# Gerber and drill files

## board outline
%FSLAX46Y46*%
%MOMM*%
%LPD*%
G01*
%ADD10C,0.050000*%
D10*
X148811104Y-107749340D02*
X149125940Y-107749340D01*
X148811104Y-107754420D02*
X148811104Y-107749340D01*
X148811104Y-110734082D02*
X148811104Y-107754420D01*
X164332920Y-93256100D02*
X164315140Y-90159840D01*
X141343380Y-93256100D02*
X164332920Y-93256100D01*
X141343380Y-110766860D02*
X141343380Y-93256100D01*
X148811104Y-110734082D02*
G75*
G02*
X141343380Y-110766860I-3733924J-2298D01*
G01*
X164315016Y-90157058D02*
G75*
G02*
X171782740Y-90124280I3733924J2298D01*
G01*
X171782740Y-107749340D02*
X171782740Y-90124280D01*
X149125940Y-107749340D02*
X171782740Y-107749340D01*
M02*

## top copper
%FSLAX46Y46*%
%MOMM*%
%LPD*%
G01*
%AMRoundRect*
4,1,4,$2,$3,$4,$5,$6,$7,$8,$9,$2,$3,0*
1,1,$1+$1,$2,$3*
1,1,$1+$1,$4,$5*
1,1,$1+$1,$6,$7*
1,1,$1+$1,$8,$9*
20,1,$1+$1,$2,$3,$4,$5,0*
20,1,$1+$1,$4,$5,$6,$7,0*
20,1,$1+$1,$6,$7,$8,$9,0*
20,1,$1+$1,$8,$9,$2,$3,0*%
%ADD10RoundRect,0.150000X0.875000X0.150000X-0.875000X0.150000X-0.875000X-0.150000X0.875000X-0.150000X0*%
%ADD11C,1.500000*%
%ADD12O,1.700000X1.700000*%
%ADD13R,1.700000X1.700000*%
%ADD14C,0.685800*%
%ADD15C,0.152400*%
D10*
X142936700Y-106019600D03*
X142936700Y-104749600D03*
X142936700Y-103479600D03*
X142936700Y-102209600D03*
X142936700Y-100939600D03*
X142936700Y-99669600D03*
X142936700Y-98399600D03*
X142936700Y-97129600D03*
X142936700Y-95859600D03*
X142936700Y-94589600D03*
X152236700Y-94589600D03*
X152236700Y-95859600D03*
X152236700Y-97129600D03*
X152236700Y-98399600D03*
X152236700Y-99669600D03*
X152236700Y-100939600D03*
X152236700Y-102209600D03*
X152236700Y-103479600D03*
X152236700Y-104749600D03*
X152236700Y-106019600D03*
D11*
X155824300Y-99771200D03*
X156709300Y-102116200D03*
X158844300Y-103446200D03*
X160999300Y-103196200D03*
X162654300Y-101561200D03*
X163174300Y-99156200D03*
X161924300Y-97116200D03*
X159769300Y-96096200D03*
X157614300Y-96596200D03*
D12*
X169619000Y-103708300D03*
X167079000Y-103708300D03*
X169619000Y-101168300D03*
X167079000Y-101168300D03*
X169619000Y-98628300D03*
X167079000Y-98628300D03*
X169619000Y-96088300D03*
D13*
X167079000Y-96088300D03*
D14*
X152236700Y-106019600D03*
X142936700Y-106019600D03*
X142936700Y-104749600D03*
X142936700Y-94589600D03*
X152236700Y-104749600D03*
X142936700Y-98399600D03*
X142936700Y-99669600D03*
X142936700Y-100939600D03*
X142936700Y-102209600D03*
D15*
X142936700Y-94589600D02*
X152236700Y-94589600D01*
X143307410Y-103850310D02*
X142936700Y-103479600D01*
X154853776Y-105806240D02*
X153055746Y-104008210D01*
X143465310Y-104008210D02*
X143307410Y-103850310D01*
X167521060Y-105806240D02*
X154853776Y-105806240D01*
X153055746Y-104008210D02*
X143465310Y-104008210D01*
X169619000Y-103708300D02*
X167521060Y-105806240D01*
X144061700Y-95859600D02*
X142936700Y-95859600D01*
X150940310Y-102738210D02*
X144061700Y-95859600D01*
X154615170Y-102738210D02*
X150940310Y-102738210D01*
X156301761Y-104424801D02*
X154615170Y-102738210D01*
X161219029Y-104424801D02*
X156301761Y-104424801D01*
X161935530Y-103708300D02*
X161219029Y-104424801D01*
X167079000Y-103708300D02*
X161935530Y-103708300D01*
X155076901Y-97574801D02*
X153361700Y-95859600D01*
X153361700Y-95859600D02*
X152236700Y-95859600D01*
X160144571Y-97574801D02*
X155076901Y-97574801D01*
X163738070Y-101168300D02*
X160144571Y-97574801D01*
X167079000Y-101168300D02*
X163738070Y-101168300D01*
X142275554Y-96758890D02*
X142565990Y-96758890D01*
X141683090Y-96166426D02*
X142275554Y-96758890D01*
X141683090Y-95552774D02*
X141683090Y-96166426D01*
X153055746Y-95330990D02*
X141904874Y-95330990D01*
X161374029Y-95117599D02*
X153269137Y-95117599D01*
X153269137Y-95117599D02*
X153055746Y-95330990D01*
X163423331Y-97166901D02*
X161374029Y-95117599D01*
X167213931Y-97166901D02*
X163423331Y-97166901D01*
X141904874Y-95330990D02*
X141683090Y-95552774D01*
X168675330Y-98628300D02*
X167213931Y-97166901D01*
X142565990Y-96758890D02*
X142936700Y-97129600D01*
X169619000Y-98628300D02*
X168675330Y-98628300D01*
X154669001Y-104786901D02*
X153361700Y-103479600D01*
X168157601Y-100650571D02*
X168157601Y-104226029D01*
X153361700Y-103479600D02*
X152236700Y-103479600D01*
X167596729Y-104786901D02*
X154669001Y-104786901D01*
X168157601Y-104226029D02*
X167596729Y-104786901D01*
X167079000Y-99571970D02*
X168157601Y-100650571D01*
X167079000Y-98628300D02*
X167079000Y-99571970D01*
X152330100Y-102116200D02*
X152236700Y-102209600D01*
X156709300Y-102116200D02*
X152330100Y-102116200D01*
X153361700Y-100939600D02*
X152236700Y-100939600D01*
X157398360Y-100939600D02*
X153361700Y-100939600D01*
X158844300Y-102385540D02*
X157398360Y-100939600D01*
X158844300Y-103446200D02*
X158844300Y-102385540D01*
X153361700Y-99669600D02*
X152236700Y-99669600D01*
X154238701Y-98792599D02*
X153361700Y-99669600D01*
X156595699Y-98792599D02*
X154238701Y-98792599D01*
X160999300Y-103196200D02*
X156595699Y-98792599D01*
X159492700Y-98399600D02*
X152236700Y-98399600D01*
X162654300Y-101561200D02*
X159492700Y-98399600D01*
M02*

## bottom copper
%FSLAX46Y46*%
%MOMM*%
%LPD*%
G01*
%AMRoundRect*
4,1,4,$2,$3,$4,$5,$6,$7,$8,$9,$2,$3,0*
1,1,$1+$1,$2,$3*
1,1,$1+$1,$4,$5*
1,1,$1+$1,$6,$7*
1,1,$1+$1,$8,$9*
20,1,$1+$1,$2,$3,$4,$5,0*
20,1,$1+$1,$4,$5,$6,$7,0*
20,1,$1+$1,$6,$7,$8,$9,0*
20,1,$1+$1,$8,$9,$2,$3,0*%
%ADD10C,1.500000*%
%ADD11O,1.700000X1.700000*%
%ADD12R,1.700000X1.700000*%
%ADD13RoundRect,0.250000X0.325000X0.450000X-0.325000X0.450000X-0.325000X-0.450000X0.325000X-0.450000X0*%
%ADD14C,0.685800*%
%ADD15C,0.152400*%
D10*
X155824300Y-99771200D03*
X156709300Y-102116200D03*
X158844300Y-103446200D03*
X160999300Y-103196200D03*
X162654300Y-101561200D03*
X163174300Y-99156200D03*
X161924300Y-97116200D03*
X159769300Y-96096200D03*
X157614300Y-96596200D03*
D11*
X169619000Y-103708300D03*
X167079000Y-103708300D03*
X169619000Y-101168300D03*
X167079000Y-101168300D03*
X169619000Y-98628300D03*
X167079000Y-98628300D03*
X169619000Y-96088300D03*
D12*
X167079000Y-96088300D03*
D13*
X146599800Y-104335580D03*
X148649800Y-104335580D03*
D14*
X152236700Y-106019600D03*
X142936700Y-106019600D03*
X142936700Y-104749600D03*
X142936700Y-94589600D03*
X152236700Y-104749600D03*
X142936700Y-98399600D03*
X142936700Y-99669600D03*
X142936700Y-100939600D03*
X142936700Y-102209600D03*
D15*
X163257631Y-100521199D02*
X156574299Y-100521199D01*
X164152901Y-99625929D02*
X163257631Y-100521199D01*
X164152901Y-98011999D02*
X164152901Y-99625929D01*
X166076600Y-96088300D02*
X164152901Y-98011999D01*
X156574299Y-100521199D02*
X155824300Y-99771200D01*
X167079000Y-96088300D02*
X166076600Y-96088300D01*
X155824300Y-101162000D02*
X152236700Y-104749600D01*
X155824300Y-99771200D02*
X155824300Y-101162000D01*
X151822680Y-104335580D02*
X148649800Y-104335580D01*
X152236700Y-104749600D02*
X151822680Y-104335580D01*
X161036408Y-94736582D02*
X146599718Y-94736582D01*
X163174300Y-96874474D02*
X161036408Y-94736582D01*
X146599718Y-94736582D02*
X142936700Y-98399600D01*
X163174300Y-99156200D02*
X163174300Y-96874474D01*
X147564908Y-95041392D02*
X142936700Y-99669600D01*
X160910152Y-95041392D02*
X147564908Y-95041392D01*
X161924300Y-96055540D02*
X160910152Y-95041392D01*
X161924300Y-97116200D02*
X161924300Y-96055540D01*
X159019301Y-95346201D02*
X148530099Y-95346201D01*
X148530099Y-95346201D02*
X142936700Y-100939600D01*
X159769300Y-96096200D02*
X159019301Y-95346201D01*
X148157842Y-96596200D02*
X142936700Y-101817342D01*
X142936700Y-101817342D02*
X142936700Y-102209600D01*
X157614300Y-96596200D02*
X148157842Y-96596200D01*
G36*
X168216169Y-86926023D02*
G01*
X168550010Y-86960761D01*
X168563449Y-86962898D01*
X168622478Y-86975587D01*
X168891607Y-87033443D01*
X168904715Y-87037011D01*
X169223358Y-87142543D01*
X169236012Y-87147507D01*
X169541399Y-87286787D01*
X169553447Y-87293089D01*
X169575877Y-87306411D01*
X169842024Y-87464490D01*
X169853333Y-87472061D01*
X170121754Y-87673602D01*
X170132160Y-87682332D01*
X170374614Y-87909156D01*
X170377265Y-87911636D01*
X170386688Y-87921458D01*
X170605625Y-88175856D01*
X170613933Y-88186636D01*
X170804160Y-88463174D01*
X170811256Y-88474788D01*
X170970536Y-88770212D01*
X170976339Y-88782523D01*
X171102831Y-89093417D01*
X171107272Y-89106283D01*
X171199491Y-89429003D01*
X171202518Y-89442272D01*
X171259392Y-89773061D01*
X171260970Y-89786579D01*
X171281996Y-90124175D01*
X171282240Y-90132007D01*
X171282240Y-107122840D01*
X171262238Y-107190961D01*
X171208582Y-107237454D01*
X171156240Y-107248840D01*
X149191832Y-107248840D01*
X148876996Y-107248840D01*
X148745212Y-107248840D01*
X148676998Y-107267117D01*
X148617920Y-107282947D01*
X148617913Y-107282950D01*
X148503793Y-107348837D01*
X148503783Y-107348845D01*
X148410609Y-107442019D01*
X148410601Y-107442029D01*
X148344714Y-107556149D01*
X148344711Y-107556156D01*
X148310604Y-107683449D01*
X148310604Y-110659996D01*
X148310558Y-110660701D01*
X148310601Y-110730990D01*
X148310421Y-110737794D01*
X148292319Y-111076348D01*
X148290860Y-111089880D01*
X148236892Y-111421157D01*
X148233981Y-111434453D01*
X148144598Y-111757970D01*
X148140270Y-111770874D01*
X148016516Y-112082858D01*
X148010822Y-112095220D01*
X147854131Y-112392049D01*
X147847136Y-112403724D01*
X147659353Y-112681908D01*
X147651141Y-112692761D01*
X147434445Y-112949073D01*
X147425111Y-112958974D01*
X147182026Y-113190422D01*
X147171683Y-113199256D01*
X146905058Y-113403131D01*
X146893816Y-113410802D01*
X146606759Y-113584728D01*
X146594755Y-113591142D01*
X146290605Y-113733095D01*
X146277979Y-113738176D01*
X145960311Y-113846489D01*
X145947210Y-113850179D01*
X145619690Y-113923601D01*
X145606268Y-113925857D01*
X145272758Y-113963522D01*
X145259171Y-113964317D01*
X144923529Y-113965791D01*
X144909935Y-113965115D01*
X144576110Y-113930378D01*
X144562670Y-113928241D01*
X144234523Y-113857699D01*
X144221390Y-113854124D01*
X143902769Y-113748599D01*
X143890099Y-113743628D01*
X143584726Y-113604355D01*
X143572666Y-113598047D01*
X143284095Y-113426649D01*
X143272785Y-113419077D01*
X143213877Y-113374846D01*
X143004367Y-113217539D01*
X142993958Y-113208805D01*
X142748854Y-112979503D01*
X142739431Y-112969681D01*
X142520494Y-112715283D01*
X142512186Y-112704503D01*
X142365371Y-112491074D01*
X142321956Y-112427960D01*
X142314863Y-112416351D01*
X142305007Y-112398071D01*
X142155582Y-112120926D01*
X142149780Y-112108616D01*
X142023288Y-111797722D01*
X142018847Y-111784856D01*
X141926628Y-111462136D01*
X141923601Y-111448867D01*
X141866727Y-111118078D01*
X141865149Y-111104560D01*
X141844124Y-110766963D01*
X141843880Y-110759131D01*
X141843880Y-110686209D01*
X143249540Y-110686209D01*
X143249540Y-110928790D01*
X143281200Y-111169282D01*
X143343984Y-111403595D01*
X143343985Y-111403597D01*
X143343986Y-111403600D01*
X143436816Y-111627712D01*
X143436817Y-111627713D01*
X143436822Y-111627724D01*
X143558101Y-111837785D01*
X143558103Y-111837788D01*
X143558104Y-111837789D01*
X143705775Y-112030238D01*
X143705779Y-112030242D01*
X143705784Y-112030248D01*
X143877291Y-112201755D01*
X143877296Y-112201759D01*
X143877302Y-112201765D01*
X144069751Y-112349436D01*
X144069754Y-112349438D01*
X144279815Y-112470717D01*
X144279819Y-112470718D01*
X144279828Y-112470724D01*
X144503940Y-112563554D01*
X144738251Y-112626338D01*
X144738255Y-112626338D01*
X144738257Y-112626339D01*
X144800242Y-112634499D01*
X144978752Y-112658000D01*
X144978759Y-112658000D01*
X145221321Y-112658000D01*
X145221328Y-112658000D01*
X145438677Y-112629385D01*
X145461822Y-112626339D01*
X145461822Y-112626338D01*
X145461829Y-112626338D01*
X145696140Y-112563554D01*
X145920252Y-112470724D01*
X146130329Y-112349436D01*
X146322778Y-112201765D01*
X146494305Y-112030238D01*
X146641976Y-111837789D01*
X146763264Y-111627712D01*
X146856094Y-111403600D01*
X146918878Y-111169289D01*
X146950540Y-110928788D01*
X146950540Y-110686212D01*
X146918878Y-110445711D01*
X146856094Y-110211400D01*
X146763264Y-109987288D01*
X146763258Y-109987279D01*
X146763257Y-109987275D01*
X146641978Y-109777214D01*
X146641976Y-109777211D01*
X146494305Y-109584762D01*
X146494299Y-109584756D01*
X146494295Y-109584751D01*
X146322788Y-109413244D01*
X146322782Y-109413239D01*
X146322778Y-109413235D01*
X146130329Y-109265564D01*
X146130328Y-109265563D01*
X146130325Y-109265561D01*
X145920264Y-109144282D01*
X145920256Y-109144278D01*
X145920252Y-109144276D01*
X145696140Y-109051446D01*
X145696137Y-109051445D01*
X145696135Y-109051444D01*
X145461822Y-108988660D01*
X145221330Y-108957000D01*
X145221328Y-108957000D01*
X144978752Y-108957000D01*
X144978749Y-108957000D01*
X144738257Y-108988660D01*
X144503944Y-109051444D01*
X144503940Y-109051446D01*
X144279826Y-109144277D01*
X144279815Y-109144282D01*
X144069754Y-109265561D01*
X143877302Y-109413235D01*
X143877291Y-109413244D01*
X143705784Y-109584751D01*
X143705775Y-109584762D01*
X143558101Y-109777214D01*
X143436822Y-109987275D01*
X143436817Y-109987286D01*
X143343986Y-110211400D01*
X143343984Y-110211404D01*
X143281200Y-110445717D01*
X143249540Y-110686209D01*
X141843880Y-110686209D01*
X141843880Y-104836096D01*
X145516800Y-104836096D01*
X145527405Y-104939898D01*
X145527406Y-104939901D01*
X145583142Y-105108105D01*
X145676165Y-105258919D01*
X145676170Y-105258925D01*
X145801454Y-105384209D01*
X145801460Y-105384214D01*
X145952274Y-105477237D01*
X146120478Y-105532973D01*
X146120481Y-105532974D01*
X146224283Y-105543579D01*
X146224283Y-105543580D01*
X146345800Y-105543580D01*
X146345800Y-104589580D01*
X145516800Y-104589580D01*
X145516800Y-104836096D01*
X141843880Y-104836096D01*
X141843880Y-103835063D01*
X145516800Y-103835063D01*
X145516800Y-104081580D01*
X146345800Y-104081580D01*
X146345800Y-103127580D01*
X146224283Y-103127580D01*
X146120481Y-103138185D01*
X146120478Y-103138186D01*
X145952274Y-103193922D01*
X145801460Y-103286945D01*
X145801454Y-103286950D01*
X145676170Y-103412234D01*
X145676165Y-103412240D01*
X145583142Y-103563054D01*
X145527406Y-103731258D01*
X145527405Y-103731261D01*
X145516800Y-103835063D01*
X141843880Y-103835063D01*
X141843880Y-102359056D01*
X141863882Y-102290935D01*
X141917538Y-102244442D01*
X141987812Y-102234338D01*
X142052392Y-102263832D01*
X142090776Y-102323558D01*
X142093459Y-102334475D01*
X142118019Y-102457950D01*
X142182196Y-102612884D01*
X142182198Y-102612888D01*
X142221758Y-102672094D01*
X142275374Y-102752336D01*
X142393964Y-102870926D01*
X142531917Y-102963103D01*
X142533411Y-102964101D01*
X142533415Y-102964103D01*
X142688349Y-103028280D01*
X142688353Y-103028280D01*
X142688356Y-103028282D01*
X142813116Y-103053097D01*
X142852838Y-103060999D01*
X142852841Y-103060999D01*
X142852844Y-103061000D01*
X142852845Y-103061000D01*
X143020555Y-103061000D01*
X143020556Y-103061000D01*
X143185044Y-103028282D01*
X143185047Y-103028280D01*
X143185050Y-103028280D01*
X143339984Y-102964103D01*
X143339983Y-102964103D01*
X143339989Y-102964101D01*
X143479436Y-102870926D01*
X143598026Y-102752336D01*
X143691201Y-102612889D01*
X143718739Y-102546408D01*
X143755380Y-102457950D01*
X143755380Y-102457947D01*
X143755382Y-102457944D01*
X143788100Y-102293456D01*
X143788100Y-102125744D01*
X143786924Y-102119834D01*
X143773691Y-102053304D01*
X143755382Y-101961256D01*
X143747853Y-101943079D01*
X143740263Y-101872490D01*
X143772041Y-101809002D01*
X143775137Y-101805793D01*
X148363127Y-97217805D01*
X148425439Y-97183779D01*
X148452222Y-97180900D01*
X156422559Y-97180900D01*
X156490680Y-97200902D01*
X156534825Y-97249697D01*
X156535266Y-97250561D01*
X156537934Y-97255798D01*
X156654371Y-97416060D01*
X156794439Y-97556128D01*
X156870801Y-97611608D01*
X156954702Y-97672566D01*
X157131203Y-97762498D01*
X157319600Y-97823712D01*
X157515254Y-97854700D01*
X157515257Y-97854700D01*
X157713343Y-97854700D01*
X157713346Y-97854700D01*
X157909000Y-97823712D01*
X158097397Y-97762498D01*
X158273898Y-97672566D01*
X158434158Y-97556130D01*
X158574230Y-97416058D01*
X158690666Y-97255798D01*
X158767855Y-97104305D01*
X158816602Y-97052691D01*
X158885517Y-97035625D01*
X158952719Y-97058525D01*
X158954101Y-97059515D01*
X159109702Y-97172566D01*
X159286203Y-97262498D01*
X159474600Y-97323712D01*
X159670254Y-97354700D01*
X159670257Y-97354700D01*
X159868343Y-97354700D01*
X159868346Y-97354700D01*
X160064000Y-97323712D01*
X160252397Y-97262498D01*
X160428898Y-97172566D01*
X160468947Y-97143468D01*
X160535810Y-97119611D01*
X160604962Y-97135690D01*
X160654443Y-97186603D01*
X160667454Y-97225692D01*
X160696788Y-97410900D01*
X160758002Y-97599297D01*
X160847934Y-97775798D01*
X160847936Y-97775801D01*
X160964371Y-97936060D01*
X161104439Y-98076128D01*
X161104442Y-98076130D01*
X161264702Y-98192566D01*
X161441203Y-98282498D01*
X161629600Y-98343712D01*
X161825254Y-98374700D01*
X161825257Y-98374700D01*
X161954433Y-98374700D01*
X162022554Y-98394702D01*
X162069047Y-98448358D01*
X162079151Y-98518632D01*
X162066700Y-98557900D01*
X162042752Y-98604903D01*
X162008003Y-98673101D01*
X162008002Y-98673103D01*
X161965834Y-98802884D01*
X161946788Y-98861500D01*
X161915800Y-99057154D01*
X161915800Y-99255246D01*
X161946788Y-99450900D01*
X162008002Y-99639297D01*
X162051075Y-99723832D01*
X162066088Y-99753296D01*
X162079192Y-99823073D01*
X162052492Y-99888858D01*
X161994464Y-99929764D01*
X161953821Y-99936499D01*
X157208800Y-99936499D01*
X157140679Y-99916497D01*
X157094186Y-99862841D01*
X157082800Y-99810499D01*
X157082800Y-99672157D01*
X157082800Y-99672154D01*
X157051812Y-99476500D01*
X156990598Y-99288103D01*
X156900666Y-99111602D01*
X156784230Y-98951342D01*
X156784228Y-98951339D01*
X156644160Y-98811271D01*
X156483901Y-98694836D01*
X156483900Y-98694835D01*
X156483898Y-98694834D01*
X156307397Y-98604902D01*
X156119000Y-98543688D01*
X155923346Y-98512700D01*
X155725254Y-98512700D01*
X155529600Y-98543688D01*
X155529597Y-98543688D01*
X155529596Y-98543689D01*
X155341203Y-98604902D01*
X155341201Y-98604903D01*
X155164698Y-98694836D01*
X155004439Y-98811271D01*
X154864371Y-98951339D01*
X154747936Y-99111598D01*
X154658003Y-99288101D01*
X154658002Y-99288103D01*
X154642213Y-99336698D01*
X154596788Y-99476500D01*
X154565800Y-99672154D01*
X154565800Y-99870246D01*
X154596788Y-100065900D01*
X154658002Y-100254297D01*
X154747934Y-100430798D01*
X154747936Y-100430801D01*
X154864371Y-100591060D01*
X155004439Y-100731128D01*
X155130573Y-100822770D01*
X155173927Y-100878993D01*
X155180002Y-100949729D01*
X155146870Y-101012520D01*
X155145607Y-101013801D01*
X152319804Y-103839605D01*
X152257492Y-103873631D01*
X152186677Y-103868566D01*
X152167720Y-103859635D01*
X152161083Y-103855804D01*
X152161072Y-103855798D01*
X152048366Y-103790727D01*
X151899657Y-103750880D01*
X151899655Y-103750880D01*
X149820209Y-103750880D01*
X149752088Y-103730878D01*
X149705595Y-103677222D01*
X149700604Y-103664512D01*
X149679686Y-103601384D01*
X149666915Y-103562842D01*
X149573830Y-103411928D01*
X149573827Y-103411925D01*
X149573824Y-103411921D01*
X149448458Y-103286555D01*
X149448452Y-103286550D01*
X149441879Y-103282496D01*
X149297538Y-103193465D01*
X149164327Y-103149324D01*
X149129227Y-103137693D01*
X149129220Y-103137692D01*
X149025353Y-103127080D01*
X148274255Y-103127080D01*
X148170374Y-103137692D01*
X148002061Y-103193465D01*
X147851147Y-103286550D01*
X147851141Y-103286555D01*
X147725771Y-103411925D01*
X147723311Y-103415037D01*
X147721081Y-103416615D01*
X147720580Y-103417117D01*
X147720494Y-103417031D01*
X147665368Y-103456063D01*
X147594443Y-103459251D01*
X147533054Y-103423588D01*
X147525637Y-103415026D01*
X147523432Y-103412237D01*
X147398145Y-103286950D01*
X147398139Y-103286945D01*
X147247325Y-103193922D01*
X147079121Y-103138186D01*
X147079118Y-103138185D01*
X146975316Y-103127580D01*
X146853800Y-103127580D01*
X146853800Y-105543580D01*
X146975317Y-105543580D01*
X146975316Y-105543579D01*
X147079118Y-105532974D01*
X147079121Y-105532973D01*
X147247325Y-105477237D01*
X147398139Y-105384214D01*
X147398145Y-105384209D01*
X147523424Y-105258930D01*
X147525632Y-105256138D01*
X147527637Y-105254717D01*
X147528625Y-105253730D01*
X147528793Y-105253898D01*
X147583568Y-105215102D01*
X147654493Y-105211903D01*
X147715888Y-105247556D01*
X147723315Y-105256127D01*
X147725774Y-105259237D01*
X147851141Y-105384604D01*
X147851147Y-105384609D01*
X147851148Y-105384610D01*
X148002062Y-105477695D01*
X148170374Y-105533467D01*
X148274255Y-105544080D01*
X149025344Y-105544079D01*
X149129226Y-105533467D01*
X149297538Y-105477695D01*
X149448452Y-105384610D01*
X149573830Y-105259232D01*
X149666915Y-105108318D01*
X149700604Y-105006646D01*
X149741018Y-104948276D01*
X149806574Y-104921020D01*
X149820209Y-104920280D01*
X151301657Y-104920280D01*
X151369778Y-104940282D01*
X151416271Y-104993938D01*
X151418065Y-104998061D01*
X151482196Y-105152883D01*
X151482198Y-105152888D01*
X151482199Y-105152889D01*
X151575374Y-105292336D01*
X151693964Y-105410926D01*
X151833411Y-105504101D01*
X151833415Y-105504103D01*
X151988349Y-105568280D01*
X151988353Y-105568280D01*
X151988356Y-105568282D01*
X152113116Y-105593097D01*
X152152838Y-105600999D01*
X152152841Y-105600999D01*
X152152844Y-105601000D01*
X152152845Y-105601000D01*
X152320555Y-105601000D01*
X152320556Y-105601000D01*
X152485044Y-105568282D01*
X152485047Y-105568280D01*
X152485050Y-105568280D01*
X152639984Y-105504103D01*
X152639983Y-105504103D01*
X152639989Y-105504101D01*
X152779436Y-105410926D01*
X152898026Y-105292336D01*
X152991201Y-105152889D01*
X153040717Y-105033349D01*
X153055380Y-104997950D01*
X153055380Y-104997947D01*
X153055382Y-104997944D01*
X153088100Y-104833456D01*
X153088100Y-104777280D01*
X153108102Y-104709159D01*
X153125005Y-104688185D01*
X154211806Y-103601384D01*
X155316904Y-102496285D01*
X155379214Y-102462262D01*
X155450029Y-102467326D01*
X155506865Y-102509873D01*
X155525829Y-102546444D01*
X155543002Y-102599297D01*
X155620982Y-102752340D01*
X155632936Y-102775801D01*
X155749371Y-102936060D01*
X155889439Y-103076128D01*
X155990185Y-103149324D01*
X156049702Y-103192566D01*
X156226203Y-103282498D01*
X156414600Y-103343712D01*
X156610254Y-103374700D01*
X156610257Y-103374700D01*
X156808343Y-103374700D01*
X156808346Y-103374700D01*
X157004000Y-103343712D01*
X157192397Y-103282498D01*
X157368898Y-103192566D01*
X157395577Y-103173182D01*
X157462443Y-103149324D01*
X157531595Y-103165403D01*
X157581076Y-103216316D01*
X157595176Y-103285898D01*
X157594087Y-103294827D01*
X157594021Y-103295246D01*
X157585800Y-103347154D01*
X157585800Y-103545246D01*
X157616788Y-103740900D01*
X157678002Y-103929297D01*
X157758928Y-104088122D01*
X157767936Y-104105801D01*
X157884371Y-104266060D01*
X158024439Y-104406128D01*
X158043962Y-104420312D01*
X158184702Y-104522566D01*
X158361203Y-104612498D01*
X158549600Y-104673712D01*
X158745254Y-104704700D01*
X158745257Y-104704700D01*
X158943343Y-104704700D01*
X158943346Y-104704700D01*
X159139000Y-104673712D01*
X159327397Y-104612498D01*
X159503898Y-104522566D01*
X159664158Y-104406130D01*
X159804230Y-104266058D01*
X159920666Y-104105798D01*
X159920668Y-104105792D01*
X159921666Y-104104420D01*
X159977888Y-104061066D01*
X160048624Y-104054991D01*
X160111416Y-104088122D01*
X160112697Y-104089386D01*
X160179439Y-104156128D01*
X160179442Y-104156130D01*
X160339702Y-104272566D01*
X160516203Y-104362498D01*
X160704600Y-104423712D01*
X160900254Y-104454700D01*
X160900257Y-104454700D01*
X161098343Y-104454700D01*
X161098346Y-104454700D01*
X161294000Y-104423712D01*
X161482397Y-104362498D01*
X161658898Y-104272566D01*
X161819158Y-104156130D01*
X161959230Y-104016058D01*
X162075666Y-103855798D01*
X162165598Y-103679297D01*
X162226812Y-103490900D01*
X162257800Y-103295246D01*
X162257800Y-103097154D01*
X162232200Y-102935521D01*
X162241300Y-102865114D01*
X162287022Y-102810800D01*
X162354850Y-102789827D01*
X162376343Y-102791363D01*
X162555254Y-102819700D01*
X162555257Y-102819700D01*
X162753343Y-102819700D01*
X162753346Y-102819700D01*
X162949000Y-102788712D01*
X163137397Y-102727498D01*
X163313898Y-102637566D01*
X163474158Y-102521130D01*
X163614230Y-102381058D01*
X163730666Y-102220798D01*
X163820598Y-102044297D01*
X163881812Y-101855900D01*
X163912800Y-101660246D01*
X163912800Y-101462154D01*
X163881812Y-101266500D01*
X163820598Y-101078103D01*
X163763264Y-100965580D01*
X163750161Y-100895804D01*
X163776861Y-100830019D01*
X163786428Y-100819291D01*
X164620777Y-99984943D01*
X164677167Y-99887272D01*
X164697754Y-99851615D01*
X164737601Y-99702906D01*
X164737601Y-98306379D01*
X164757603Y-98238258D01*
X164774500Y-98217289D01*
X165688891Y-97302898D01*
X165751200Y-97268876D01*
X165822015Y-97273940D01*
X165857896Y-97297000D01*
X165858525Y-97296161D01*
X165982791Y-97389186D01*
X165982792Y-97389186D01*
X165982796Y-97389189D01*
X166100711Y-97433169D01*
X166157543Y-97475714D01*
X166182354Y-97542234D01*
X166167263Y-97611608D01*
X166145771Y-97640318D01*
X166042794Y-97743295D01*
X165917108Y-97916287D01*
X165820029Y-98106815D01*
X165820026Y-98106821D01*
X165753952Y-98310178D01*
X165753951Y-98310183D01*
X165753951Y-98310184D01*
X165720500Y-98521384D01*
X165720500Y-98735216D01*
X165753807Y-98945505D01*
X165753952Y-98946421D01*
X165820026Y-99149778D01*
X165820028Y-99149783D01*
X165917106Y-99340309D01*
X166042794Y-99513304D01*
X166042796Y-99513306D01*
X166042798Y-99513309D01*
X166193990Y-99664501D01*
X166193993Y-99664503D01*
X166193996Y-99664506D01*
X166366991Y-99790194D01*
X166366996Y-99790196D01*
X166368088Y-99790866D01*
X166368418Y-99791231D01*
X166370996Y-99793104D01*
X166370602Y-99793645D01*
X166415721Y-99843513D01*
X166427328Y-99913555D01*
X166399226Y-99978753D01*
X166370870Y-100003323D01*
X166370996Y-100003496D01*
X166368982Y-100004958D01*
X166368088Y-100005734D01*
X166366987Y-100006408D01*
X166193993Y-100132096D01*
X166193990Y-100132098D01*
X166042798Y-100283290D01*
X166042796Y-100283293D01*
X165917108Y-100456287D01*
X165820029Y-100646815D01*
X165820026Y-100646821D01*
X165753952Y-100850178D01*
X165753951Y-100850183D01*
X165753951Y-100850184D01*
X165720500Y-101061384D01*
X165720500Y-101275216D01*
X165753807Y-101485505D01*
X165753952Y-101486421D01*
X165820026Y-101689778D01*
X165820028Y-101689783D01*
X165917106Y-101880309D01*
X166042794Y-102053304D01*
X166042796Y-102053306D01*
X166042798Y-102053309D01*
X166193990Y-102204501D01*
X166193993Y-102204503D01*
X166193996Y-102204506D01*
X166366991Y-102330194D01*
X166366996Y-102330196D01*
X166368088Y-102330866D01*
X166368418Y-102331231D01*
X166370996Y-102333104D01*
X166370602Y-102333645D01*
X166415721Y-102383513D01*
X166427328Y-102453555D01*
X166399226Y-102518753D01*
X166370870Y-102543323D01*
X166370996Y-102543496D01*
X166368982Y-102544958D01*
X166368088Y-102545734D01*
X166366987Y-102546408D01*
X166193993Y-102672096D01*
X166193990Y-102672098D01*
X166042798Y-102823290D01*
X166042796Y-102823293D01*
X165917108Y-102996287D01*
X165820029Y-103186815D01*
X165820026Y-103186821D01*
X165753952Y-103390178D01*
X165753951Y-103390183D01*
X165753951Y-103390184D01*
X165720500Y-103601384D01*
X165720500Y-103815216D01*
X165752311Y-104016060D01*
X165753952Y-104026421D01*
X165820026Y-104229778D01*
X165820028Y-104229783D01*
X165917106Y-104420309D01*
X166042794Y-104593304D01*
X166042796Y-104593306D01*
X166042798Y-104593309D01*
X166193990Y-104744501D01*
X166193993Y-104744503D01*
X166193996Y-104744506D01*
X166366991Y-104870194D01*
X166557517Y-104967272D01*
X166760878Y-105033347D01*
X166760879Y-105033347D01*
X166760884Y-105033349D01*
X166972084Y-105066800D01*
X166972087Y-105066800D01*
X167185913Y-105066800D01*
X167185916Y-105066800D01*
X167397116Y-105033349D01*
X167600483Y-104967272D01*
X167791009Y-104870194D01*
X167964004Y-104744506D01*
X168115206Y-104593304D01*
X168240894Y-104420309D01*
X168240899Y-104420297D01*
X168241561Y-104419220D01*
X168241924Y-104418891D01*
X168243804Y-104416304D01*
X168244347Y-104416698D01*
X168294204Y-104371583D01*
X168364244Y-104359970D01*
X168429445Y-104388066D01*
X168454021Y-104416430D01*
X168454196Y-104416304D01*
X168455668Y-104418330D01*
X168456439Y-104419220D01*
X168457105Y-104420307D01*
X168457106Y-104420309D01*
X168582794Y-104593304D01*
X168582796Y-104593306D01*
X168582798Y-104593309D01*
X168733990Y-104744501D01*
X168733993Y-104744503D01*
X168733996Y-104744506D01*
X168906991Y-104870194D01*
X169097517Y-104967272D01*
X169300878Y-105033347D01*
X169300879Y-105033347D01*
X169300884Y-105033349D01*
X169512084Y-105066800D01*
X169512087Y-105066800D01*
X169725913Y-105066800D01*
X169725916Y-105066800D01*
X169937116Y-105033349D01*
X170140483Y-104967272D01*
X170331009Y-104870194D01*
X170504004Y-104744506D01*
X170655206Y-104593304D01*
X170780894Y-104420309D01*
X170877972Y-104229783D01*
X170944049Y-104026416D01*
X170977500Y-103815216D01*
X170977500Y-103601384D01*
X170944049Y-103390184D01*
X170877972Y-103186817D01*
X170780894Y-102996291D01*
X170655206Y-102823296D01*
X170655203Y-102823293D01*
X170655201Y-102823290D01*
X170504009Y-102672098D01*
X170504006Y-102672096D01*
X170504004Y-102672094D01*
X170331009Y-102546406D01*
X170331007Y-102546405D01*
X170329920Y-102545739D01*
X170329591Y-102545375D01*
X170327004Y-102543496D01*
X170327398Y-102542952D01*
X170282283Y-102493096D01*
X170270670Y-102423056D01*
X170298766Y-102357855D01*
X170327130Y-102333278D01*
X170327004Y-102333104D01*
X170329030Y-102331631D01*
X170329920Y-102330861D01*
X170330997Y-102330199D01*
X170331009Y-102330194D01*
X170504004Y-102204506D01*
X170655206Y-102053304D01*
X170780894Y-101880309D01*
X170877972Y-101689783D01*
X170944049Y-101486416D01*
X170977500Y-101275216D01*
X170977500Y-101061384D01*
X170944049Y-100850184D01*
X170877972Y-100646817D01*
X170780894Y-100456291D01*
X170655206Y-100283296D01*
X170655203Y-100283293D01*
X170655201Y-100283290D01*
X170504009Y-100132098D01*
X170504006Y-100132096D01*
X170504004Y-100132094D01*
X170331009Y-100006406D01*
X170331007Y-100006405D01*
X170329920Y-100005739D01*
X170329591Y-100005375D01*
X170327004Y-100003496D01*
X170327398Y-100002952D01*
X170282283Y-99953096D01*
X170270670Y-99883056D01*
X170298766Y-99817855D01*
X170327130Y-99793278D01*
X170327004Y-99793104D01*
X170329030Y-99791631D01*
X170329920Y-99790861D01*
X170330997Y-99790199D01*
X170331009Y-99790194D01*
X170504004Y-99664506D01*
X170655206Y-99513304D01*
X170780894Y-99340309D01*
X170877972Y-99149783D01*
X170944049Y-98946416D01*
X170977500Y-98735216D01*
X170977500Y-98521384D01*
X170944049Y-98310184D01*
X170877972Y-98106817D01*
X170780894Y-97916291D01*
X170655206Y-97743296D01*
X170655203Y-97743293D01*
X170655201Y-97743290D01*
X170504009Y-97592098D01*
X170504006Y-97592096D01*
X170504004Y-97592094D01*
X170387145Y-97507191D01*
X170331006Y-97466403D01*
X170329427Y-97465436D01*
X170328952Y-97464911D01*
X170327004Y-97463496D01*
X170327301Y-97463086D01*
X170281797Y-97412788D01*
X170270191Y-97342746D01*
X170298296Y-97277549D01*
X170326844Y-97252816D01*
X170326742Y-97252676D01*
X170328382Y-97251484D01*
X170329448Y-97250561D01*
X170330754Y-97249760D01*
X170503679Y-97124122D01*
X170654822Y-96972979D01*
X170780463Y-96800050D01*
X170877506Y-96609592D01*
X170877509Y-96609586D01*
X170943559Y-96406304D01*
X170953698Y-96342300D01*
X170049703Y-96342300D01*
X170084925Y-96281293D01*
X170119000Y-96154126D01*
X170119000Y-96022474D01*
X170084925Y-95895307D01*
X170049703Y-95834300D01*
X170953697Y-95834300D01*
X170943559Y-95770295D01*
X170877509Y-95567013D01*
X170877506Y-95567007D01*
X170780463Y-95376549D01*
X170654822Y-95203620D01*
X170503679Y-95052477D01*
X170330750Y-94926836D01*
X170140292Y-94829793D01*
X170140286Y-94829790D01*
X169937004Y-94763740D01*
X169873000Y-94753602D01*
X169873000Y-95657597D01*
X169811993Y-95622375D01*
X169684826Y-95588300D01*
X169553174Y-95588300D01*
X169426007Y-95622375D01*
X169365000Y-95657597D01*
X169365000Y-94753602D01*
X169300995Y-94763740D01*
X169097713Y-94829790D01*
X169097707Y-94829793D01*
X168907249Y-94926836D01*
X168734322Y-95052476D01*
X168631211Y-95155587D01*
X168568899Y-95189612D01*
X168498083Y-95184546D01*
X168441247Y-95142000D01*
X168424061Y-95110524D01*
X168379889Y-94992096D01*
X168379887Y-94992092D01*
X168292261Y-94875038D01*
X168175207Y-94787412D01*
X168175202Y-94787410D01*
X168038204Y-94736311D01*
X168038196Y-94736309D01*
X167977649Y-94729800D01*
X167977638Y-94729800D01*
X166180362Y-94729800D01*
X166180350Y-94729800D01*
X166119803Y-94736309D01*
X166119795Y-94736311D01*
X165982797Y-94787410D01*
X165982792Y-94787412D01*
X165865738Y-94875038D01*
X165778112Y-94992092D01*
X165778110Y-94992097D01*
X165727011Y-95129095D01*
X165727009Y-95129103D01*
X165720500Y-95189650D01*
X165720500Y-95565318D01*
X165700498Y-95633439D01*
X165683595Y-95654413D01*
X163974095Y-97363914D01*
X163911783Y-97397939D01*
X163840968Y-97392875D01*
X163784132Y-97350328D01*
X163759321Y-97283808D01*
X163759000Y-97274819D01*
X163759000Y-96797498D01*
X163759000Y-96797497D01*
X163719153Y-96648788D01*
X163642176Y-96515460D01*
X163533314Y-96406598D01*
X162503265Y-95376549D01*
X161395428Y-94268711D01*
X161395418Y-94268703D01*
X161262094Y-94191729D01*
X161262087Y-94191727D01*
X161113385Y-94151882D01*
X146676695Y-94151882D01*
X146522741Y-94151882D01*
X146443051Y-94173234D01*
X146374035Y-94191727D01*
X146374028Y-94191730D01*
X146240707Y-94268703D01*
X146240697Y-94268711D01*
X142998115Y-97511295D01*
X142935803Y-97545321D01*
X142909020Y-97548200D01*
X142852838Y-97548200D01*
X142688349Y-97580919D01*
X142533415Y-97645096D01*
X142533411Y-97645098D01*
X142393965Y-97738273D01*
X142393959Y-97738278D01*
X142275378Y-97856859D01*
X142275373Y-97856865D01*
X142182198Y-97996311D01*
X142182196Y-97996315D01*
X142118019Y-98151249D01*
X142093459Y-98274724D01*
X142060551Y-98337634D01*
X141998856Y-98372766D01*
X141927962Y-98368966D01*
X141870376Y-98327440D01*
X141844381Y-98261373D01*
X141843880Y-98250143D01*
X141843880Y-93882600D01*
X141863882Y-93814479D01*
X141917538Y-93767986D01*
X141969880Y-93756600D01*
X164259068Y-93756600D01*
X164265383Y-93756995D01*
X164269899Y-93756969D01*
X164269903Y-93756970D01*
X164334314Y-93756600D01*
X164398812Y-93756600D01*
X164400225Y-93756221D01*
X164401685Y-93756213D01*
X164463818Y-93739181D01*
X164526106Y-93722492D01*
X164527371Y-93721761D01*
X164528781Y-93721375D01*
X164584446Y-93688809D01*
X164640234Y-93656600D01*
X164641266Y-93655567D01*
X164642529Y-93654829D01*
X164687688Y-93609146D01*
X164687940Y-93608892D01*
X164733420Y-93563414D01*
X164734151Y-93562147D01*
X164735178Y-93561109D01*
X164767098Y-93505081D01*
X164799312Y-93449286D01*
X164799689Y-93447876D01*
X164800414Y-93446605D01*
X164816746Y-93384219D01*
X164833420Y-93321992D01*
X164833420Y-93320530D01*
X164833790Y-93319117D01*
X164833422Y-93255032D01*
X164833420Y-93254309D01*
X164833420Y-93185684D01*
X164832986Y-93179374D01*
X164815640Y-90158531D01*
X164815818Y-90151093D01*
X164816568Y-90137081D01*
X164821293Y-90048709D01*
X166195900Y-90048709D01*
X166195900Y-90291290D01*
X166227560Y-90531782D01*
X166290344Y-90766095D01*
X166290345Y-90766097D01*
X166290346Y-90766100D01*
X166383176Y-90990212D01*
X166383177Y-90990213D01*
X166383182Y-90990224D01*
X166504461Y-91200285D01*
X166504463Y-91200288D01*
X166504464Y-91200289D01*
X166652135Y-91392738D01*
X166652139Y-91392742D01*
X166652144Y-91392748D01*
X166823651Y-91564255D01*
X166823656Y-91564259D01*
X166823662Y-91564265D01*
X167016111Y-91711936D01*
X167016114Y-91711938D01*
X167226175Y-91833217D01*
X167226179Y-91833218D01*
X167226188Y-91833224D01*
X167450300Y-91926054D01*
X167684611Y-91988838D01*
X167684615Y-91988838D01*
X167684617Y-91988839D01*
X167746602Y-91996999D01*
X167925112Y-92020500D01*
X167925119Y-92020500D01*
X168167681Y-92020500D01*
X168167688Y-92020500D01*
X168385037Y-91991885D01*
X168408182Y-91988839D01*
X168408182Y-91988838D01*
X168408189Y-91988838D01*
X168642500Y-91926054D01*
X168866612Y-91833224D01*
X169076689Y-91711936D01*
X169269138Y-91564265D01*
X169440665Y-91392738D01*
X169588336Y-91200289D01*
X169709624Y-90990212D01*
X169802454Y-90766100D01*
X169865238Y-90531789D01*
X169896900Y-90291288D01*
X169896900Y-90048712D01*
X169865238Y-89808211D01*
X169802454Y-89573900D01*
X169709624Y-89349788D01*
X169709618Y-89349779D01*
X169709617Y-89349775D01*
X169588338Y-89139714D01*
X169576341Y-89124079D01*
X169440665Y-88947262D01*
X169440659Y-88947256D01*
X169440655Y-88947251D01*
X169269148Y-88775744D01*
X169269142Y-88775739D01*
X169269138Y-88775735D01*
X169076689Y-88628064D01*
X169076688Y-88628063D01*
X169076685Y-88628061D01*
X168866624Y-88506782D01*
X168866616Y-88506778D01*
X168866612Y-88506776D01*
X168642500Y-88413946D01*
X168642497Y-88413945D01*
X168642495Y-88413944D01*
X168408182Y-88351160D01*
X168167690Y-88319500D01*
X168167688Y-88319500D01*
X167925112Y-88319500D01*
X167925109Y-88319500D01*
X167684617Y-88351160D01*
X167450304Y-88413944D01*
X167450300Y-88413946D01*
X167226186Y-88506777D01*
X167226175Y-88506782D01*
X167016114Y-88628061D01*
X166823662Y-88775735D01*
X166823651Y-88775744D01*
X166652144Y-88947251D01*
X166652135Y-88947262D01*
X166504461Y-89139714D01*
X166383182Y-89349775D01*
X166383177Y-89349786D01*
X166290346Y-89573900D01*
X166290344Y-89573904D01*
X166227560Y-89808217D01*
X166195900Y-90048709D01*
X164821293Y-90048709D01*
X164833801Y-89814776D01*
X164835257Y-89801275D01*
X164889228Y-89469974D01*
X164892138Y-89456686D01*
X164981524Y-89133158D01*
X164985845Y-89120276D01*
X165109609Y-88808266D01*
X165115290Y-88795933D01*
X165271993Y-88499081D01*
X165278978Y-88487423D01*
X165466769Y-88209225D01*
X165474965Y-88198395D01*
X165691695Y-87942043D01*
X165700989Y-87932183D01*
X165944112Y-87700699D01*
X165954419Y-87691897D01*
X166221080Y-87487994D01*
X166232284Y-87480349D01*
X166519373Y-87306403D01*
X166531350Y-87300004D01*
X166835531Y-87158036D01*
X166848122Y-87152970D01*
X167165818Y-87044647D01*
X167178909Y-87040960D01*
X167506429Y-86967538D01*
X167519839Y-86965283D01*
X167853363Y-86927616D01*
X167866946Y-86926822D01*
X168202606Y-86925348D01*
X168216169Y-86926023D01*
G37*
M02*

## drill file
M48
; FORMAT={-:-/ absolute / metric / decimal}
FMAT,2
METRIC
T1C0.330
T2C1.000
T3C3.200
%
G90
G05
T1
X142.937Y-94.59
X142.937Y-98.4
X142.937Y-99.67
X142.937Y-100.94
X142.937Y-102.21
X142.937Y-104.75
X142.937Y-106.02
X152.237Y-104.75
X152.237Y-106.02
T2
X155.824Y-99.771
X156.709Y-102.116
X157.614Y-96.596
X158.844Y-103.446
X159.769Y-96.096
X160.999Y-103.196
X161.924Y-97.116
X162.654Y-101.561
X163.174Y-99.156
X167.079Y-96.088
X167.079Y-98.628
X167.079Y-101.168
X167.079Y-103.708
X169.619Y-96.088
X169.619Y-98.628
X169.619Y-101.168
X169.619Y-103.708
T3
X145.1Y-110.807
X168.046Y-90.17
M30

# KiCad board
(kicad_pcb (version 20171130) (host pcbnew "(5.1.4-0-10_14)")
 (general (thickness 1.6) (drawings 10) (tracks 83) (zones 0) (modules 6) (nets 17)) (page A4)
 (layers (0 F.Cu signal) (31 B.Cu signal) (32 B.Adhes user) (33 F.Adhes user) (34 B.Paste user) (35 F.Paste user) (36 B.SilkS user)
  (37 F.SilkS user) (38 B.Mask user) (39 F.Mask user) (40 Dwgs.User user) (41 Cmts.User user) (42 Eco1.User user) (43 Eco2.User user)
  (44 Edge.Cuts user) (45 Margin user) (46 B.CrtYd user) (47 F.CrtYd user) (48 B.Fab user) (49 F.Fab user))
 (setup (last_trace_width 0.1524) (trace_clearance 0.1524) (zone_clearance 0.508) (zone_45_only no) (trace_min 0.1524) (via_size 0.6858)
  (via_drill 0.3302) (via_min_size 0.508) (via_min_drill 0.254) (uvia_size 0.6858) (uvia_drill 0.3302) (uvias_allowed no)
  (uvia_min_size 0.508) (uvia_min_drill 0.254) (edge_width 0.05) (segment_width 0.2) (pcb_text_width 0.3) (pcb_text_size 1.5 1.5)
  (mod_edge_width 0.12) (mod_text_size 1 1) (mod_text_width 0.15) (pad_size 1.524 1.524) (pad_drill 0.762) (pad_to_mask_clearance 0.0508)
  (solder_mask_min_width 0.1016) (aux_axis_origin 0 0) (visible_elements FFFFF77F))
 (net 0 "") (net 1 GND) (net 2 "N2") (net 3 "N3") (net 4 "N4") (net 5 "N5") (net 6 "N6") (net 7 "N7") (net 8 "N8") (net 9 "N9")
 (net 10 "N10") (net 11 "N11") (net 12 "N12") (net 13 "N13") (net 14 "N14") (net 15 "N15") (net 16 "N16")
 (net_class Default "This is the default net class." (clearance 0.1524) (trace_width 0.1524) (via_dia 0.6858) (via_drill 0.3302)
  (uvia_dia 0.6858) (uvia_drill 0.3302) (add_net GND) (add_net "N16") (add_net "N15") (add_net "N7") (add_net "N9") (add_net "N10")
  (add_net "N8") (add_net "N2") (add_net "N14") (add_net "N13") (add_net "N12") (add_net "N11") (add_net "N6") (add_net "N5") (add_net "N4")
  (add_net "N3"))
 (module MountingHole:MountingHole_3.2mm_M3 (layer F.Cu) (at 145.10004 110.8075)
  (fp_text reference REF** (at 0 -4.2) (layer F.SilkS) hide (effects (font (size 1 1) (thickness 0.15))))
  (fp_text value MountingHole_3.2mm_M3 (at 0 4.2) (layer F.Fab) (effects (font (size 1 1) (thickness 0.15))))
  (pad 1 np_thru_hole circle (at 0 0) (size 3.2 3.2) (drill 3.2) (layers *.Cu *.Mask)))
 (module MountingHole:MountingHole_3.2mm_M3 (layer F.Cu) (at 168.0464 90.17)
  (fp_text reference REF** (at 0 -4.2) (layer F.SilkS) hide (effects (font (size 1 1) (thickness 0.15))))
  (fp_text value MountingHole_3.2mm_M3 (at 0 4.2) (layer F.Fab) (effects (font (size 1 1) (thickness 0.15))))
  (pad 1 np_thru_hole circle (at 0 0) (size 3.2 3.2) (drill 3.2) (layers *.Cu *.Mask)))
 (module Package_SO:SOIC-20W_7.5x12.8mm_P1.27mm (layer F.Cu) (at 147.5867 100.3046 180)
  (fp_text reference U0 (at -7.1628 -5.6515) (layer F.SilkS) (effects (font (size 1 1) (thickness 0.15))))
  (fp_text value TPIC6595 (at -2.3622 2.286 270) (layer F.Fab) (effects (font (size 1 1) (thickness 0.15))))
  (pad 20 smd roundrect (at 4.65 -5.715 180) (size 2.05 0.6) (layers F.Cu F.Paste F.Mask) (roundrect_rratio 0.25) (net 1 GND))
  (pad 19 smd roundrect (at 4.65 -4.445 180) (size 2.05 0.6) (layers F.Cu F.Paste F.Mask) (roundrect_rratio 0.25) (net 1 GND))
  (pad 18 smd roundrect (at 4.65 -3.175 180) (size 2.05 0.6) (layers F.Cu F.Paste F.Mask) (roundrect_rratio 0.25) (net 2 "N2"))
  (pad 17 smd roundrect (at 4.65 -1.905 180) (size 2.05 0.6) (layers F.Cu F.Paste F.Mask) (roundrect_rratio 0.25) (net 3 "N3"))
  (pad 16 smd roundrect (at 4.65 -0.635 180) (size 2.05 0.6) (layers F.Cu F.Paste F.Mask) (roundrect_rratio 0.25) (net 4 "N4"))
  (pad 15 smd roundrect (at 4.65 0.635 180) (size 2.05 0.6) (layers F.Cu F.Paste F.Mask) (roundrect_rratio 0.25) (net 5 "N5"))
  (pad 14 smd roundrect (at 4.65 1.905 180) (size 2.05 0.6) (layers F.Cu F.Paste F.Mask) (roundrect_rratio 0.25) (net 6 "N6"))
  (pad 13 smd roundrect (at 4.65 3.175 180) (size 2.05 0.6) (layers F.Cu F.Paste F.Mask) (roundrect_rratio 0.25) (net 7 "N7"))
  (pad 12 smd roundrect (at 4.65 4.445 180) (size 2.05 0.6) (layers F.Cu F.Paste F.Mask) (roundrect_rratio 0.25) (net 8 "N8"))
  (pad 11 smd roundrect (at 4.65 5.715 180) (size 2.05 0.6) (layers F.Cu F.Paste F.Mask) (roundrect_rratio 0.25) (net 1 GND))
  (pad 10 smd roundrect (at -4.65 5.715 180) (size 2.05 0.6) (layers F.Cu F.Paste F.Mask) (roundrect_rratio 0.25) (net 1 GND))
  (pad 9 smd roundrect (at -4.65 4.445 180) (size 2.05 0.6) (layers F.Cu F.Paste F.Mask) (roundrect_rratio 0.25) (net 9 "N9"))
  (pad 8 smd roundrect (at -4.65 3.175 180) (size 2.05 0.6) (layers F.Cu F.Paste F.Mask) (roundrect_rratio 0.25) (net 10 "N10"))
  (pad 7 smd roundrect (at -4.65 1.905 180) (size 2.05 0.6) (layers F.Cu F.Paste F.Mask) (roundrect_rratio 0.25) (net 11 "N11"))
  (pad 6 smd roundrect (at -4.65 0.635 180) (size 2.05 0.6) (layers F.Cu F.Paste F.Mask) (roundrect_rratio 0.25) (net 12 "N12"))
  (pad 5 smd roundrect (at -4.65 -0.635 180) (size 2.05 0.6) (layers F.Cu F.Paste F.Mask) (roundrect_rratio 0.25) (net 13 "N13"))
  (pad 4 smd roundrect (at -4.65 -1.905 180) (size 2.05 0.6) (layers F.Cu F.Paste F.Mask) (roundrect_rratio 0.25) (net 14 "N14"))
  (pad 3 smd roundrect (at -4.65 -3.175 180) (size 2.05 0.6) (layers F.Cu F.Paste F.Mask) (roundrect_rratio 0.25) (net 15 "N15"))
  (pad 2 smd roundrect (at -4.65 -4.445 180) (size 2.05 0.6) (layers F.Cu F.Paste F.Mask) (roundrect_rratio 0.25) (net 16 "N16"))
  (pad 1 smd roundrect (at -4.65 -5.715 180) (size 2.05 0.6) (layers F.Cu F.Paste F.Mask) (roundrect_rratio 0.25) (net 1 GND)))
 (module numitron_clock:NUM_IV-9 (layer F.Cu) (at 159.4993 99.7712 270)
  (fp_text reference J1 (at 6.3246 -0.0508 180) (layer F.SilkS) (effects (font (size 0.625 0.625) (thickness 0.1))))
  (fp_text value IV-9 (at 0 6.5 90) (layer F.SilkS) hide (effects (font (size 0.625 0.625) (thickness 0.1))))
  (pad 1 thru_hole circle (at 0 3.675 270) (size 1.5 1.5) (drill 1) (layers *.Cu *.Mask F.SilkS) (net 16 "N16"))
  (pad 2 thru_hole circle (at 2.345 2.79 270) (size 1.5 1.5) (drill 1) (layers *.Cu *.Mask F.SilkS) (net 14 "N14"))
  (pad 3 thru_hole circle (at 3.675 0.655 270) (size 1.5 1.5) (drill 1) (layers *.Cu *.Mask F.SilkS) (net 13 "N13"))
  (pad 4 thru_hole circle (at 3.425 -1.5 270) (size 1.5 1.5) (drill 1) (layers *.Cu *.Mask F.SilkS) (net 12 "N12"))
  (pad 5 thru_hole circle (at 1.79 -3.155 270) (size 1.5 1.5) (drill 1) (layers *.Cu *.Mask F.SilkS) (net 11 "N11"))
  (pad 6 thru_hole circle (at -0.615 -3.675 270) (size 1.5 1.5) (drill 1) (layers *.Cu *.Mask F.SilkS) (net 6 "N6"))
  (pad 7 thru_hole circle (at -2.655 -2.425 270) (size 1.5 1.5) (drill 1) (layers *.Cu *.Mask F.SilkS) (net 5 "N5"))
  (pad 8 thru_hole circle (at -3.675 -0.27 270) (size 1.5 1.5) (drill 1) (layers *.Cu *.Mask F.SilkS) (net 4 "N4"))
  (pad 9 thru_hole circle (at -3.175 1.885 270) (size 1.5 1.5) (drill 1) (layers *.Cu *.Mask F.SilkS) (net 3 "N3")))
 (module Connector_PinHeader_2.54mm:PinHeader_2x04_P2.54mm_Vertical (layer F.Cu) (at 167.079 96.0883)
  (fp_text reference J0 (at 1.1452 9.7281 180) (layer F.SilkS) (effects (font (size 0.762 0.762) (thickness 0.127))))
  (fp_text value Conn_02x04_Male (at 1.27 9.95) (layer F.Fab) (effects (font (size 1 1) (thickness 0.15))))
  (pad 8 thru_hole oval (at 2.54 7.62) (size 1.7 1.7) (drill 1) (layers *.Cu *.Mask) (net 2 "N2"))
  (pad 7 thru_hole oval (at 0 7.62) (size 1.7 1.7) (drill 1) (layers *.Cu *.Mask) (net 8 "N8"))
  (pad 6 thru_hole oval (at 2.54 5.08) (size 1.7 1.7) (drill 1) (layers *.Cu *.Mask) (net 10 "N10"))
  (pad 5 thru_hole oval (at 0 5.08) (size 1.7 1.7) (drill 1) (layers *.Cu *.Mask) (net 9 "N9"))
  (pad 4 thru_hole oval (at 2.54 2.54) (size 1.7 1.7) (drill 1) (layers *.Cu *.Mask) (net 7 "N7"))
  (pad 3 thru_hole oval (at 0 2.54) (size 1.7 1.7) (drill 1) (layers *.Cu *.Mask) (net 15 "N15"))
  (pad 2 thru_hole oval (at 2.54 0) (size 1.7 1.7) (drill 1) (layers *.Cu *.Mask) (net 1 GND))
  (pad 1 thru_hole rect (at 0 0) (size 1.7 1.7) (drill 1) (layers *.Cu *.Mask) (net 16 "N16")))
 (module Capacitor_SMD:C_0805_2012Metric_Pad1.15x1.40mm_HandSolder (layer B.Cu) (at 147.6248 104.33558 180)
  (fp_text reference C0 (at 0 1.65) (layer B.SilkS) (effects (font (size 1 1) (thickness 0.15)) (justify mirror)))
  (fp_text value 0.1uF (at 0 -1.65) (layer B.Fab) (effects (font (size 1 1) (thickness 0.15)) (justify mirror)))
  (pad 2 smd roundrect (at 1.025 0 180) (size 1.15 1.4) (layers B.Cu B.Paste B.Mask) (roundrect_rratio 0.217391) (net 1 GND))
  (pad 1 smd roundrect (at -1.025 0 180) (size 1.15 1.4) (layers B.Cu B.Paste B.Mask) (roundrect_rratio 0.217391) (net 16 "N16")))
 (gr_line (start 148.811104 107.74934) (end 149.12594 107.74934) (layer Edge.Cuts) (width 0.05))
 (gr_line (start 148.811104 107.75442) (end 148.811104 107.74934) (layer Edge.Cuts) (width 0.05))
 (gr_line (start 148.811104 110.734082) (end 148.811104 107.75442) (layer Edge.Cuts) (width 0.05))
 (gr_line (start 164.33292 93.2561) (end 164.31514 90.15984) (layer Edge.Cuts) (width 0.05))
 (gr_line (start 141.34338 93.2561) (end 164.33292 93.2561) (layer Edge.Cuts) (width 0.05))
 (gr_line (start 141.34338 110.76686) (end 141.34338 93.2561) (layer Edge.Cuts) (width 0.05))
 (gr_arc (start 145.07718 110.73638) (end 141.34338 110.76686) (angle -179.567545) (layer Edge.Cuts) (width 0.05))
 (gr_arc (start 168.04894 90.15476) (end 171.78274 90.12428) (angle -179.567545) (layer Edge.Cuts) (width 0.05))
 (gr_line (start 171.78274 107.74934) (end 171.78274 90.12428) (layer Edge.Cuts) (width 0.05))
 (gr_line (start 149.12594 107.74934) (end 171.78274 107.74934) (layer Edge.Cuts) (width 0.05))
 (via (at 152.2367 106.0196) (size 0.6858) (drill 0.3302) (layers F.Cu B.Cu) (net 1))
 (via (at 142.9367 106.0196) (size 0.6858) (drill 0.3302) (layers F.Cu B.Cu) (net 1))
 (via (at 142.9367 104.7496) (size 0.6858) (drill 0.3302) (layers F.Cu B.Cu) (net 1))
 (via (at 142.9367 94.5896) (size 0.6858) (drill 0.3302) (layers F.Cu B.Cu) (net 1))
 (segment (start 142.9367 94.5896) (end 152.2367 94.5896) (width 0.1524) (layer F.Cu) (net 1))
 (via (at 152.2367 104.7496) (size 0.6858) (drill 0.3302) (layers F.Cu B.Cu) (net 16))
 (segment (start 163.257631 100.521199) (end 156.574299 100.521199) (width 0.1524) (layer B.Cu) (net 16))
 (segment (start 164.152901 99.625929) (end 163.257631 100.521199) (width 0.1524) (layer B.Cu) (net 16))
 (segment (start 164.152901 98.011999) (end 164.152901 99.625929) (width 0.1524) (layer B.Cu) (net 16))
 (segment (start 166.0766 96.0883) (end 164.152901 98.011999) (width 0.1524) (layer B.Cu) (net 16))
 (segment (start 156.574299 100.521199) (end 155.8243 99.7712) (width 0.1524) (layer B.Cu) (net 16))
 (segment (start 167.079 96.0883) (end 166.0766 96.0883) (width 0.1524) (layer B.Cu) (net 16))
 (segment (start 155.8243 101.162) (end 152.2367 104.7496) (width 0.1524) (layer B.Cu) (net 16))
 (segment (start 155.8243 99.7712) (end 155.8243 101.162) (width 0.1524) (layer B.Cu) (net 16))
 (segment (start 151.82268 104.33558) (end 148.6498 104.33558) (width 0.1524) (layer B.Cu) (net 16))
 (segment (start 152.2367 104.7496) (end 151.82268 104.33558) (width 0.1524) (layer B.Cu) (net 16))
 (segment (start 143.30741 103.85031) (end 142.9367 103.4796) (width 0.1524) (layer F.Cu) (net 2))
 (segment (start 154.853776 105.80624) (end 153.055746 104.00821) (width 0.1524) (layer F.Cu) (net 2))
 (segment (start 143.46531 104.00821) (end 143.30741 103.85031) (width 0.1524) (layer F.Cu) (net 2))
 (segment (start 167.52106 105.80624) (end 154.853776 105.80624) (width 0.1524) (layer F.Cu) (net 2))
 (segment (start 153.055746 104.00821) (end 143.46531 104.00821) (width 0.1524) (layer F.Cu) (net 2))
 (segment (start 169.619 103.7083) (end 167.52106 105.80624) (width 0.1524) (layer F.Cu) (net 2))
 (segment (start 144.0617 95.8596) (end 142.9367 95.8596) (width 0.1524) (layer F.Cu) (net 8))
 (segment (start 150.94031 102.73821) (end 144.0617 95.8596) (width 0.1524) (layer F.Cu) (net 8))
 (segment (start 154.61517 102.73821) (end 150.94031 102.73821) (width 0.1524) (layer F.Cu) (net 8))
 (segment (start 156.301761 104.424801) (end 154.61517 102.73821) (width 0.1524) (layer F.Cu) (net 8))
 (segment (start 161.219029 104.424801) (end 156.301761 104.424801) (width 0.1524) (layer F.Cu) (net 8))
 (segment (start 161.93553 103.7083) (end 161.219029 104.424801) (width 0.1524) (layer F.Cu) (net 8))
 (segment (start 167.079 103.7083) (end 161.93553 103.7083) (width 0.1524) (layer F.Cu) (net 8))
 (segment (start 155.076901 97.574801) (end 153.3617 95.8596) (width 0.1524) (layer F.Cu) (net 9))
 (segment (start 153.3617 95.8596) (end 152.2367 95.8596) (width 0.1524) (layer F.Cu) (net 9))
 (segment (start 160.144571 97.574801) (end 155.076901 97.574801) (width 0.1524) (layer F.Cu) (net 9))
 (segment (start 163.73807 101.1683) (end 160.144571 97.574801) (width 0.1524) (layer F.Cu) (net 9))
 (segment (start 167.079 101.1683) (end 163.73807 101.1683) (width 0.1524) (layer F.Cu) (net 9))
 (segment (start 142.275554 96.75889) (end 142.56599 96.75889) (width 0.1524) (layer F.Cu) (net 7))
 (segment (start 141.68309 96.166426) (end 142.275554 96.75889) (width 0.1524) (layer F.Cu) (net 7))
 (segment (start 141.68309 95.552774) (end 141.68309 96.166426) (width 0.1524) (layer F.Cu) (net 7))
 (segment (start 153.055746 95.33099) (end 141.904874 95.33099) (width 0.1524) (layer F.Cu) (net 7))
 (segment (start 161.374029 95.117599) (end 153.269137 95.117599) (width 0.1524) (layer F.Cu) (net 7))
 (segment (start 153.269137 95.117599) (end 153.055746 95.33099) (width 0.1524) (layer F.Cu) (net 7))
 (segment (start 163.423331 97.166901) (end 161.374029 95.117599) (width 0.1524) (layer F.Cu) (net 7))
 (segment (start 167.213931 97.166901) (end 163.423331 97.166901) (width 0.1524) (layer F.Cu) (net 7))
 (segment (start 141.904874 95.33099) (end 141.68309 95.552774) (width 0.1524) (layer F.Cu) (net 7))
 (segment (start 168.67533 98.6283) (end 167.213931 97.166901) (width 0.1524) (layer F.Cu) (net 7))
 (segment (start 142.56599 96.75889) (end 142.9367 97.1296) (width 0.1524) (layer F.Cu) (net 7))
 (segment (start 169.619 98.6283) (end 168.67533 98.6283) (width 0.1524) (layer F.Cu) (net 7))
 (segment (start 154.669001 104.786901) (end 153.3617 103.4796) (width 0.1524) (layer F.Cu) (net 15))
 (segment (start 168.157601 100.650571) (end 168.157601 104.226029) (width 0.1524) (layer F.Cu) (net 15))
 (segment (start 153.3617 103.4796) (end 152.2367 103.4796) (width 0.1524) (layer F.Cu) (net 15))
 (segment (start 167.596729 104.786901) (end 154.669001 104.786901) (width 0.1524) (layer F.Cu) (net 15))
 (segment (start 168.157601 104.226029) (end 167.596729 104.786901) (width 0.1524) (layer F.Cu) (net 15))
 (segment (start 167.079 99.57197) (end 168.157601 100.650571) (width 0.1524) (layer F.Cu) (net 15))
 (segment (start 167.079 98.6283) (end 167.079 99.57197) (width 0.1524) (layer F.Cu) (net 15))
 (segment (start 152.3301 102.1162) (end 152.2367 102.2096) (width 0.1524) (layer F.Cu) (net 14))
 (segment (start 156.7093 102.1162) (end 152.3301 102.1162) (width 0.1524) (layer F.Cu) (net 14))
 (segment (start 153.3617 100.9396) (end 152.2367 100.9396) (width 0.1524) (layer F.Cu) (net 13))
 (segment (start 157.39836 100.9396) (end 153.3617 100.9396) (width 0.1524) (layer F.Cu) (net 13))
 (segment (start 158.8443 102.38554) (end 157.39836 100.9396) (width 0.1524) (layer F.Cu) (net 13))
 (segment (start 158.8443 103.4462) (end 158.8443 102.38554) (width 0.1524) (layer F.Cu) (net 13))
 (segment (start 153.3617 99.6696) (end 152.2367 99.6696) (width 0.1524) (layer F.Cu) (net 12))
 (segment (start 154.238701 98.792599) (end 153.3617 99.6696) (width 0.1524) (layer F.Cu) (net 12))
 (segment (start 156.595699 98.792599) (end 154.238701 98.792599) (width 0.1524) (layer F.Cu) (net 12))
 (segment (start 160.9993 103.1962) (end 156.595699 98.792599) (width 0.1524) (layer F.Cu) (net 12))
 (segment (start 159.4927 98.3996) (end 152.2367 98.3996) (width 0.1524) (layer F.Cu) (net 11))
 (segment (start 162.6543 101.5612) (end 159.4927 98.3996) (width 0.1524) (layer F.Cu) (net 11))
 (segment (start 161.036408 94.736582) (end 146.599718 94.736582) (width 0.1524) (layer B.Cu) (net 6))
 (via (at 142.9367 98.3996) (size 0.6858) (drill 0.3302) (layers F.Cu B.Cu) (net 6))
 (segment (start 163.1743 96.874474) (end 161.036408 94.736582) (width 0.1524) (layer B.Cu) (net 6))
 (segment (start 146.599718 94.736582) (end 142.9367 98.3996) (width 0.1524) (layer B.Cu) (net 6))
 (segment (start 163.1743 99.1562) (end 163.1743 96.874474) (width 0.1524) (layer B.Cu) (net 6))
 (segment (start 147.564908 95.041392) (end 142.9367 99.6696) (width 0.1524) (layer B.Cu) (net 5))
 (via (at 142.9367 99.6696) (size 0.6858) (drill 0.3302) (layers F.Cu B.Cu) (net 5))
 (segment (start 160.910152 95.041392) (end 147.564908 95.041392) (width 0.1524) (layer B.Cu) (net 5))
 (segment (start 161.9243 96.05554) (end 160.910152 95.041392) (width 0.1524) (layer B.Cu) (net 5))
 (segment (start 161.9243 97.1162) (end 161.9243 96.05554) (width 0.1524) (layer B.Cu) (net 5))
 (via (at 142.9367 100.9396) (size 0.6858) (drill 0.3302) (layers F.Cu B.Cu) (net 4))
 (segment (start 159.019301 95.346201) (end 148.530099 95.346201) (width 0.1524) (layer B.Cu) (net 4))
 (segment (start 148.530099 95.346201) (end 142.9367 100.9396) (width 0.1524) (layer B.Cu) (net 4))
 (segment (start 159.7693 96.0962) (end 159.019301 95.346201) (width 0.1524) (layer B.Cu) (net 4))
 (via (at 142.9367 102.2096) (size 0.6858) (drill 0.3302) (layers F.Cu B.Cu) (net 3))
 (segment (start 148.157842 96.5962) (end 142.9367 101.817342) (width 0.1524) (layer B.Cu) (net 3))
 (segment (start 142.9367 101.817342) (end 142.9367 102.2096) (width 0.1524) (layer B.Cu) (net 3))
 (segment (start 157.6143 96.5962) (end 148.157842 96.5962) (width 0.1524) (layer B.Cu) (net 3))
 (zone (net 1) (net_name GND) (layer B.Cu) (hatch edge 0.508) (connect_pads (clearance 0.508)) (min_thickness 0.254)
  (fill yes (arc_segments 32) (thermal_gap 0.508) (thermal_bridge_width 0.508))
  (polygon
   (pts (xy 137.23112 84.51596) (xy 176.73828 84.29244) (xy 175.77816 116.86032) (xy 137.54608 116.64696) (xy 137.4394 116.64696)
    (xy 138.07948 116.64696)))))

